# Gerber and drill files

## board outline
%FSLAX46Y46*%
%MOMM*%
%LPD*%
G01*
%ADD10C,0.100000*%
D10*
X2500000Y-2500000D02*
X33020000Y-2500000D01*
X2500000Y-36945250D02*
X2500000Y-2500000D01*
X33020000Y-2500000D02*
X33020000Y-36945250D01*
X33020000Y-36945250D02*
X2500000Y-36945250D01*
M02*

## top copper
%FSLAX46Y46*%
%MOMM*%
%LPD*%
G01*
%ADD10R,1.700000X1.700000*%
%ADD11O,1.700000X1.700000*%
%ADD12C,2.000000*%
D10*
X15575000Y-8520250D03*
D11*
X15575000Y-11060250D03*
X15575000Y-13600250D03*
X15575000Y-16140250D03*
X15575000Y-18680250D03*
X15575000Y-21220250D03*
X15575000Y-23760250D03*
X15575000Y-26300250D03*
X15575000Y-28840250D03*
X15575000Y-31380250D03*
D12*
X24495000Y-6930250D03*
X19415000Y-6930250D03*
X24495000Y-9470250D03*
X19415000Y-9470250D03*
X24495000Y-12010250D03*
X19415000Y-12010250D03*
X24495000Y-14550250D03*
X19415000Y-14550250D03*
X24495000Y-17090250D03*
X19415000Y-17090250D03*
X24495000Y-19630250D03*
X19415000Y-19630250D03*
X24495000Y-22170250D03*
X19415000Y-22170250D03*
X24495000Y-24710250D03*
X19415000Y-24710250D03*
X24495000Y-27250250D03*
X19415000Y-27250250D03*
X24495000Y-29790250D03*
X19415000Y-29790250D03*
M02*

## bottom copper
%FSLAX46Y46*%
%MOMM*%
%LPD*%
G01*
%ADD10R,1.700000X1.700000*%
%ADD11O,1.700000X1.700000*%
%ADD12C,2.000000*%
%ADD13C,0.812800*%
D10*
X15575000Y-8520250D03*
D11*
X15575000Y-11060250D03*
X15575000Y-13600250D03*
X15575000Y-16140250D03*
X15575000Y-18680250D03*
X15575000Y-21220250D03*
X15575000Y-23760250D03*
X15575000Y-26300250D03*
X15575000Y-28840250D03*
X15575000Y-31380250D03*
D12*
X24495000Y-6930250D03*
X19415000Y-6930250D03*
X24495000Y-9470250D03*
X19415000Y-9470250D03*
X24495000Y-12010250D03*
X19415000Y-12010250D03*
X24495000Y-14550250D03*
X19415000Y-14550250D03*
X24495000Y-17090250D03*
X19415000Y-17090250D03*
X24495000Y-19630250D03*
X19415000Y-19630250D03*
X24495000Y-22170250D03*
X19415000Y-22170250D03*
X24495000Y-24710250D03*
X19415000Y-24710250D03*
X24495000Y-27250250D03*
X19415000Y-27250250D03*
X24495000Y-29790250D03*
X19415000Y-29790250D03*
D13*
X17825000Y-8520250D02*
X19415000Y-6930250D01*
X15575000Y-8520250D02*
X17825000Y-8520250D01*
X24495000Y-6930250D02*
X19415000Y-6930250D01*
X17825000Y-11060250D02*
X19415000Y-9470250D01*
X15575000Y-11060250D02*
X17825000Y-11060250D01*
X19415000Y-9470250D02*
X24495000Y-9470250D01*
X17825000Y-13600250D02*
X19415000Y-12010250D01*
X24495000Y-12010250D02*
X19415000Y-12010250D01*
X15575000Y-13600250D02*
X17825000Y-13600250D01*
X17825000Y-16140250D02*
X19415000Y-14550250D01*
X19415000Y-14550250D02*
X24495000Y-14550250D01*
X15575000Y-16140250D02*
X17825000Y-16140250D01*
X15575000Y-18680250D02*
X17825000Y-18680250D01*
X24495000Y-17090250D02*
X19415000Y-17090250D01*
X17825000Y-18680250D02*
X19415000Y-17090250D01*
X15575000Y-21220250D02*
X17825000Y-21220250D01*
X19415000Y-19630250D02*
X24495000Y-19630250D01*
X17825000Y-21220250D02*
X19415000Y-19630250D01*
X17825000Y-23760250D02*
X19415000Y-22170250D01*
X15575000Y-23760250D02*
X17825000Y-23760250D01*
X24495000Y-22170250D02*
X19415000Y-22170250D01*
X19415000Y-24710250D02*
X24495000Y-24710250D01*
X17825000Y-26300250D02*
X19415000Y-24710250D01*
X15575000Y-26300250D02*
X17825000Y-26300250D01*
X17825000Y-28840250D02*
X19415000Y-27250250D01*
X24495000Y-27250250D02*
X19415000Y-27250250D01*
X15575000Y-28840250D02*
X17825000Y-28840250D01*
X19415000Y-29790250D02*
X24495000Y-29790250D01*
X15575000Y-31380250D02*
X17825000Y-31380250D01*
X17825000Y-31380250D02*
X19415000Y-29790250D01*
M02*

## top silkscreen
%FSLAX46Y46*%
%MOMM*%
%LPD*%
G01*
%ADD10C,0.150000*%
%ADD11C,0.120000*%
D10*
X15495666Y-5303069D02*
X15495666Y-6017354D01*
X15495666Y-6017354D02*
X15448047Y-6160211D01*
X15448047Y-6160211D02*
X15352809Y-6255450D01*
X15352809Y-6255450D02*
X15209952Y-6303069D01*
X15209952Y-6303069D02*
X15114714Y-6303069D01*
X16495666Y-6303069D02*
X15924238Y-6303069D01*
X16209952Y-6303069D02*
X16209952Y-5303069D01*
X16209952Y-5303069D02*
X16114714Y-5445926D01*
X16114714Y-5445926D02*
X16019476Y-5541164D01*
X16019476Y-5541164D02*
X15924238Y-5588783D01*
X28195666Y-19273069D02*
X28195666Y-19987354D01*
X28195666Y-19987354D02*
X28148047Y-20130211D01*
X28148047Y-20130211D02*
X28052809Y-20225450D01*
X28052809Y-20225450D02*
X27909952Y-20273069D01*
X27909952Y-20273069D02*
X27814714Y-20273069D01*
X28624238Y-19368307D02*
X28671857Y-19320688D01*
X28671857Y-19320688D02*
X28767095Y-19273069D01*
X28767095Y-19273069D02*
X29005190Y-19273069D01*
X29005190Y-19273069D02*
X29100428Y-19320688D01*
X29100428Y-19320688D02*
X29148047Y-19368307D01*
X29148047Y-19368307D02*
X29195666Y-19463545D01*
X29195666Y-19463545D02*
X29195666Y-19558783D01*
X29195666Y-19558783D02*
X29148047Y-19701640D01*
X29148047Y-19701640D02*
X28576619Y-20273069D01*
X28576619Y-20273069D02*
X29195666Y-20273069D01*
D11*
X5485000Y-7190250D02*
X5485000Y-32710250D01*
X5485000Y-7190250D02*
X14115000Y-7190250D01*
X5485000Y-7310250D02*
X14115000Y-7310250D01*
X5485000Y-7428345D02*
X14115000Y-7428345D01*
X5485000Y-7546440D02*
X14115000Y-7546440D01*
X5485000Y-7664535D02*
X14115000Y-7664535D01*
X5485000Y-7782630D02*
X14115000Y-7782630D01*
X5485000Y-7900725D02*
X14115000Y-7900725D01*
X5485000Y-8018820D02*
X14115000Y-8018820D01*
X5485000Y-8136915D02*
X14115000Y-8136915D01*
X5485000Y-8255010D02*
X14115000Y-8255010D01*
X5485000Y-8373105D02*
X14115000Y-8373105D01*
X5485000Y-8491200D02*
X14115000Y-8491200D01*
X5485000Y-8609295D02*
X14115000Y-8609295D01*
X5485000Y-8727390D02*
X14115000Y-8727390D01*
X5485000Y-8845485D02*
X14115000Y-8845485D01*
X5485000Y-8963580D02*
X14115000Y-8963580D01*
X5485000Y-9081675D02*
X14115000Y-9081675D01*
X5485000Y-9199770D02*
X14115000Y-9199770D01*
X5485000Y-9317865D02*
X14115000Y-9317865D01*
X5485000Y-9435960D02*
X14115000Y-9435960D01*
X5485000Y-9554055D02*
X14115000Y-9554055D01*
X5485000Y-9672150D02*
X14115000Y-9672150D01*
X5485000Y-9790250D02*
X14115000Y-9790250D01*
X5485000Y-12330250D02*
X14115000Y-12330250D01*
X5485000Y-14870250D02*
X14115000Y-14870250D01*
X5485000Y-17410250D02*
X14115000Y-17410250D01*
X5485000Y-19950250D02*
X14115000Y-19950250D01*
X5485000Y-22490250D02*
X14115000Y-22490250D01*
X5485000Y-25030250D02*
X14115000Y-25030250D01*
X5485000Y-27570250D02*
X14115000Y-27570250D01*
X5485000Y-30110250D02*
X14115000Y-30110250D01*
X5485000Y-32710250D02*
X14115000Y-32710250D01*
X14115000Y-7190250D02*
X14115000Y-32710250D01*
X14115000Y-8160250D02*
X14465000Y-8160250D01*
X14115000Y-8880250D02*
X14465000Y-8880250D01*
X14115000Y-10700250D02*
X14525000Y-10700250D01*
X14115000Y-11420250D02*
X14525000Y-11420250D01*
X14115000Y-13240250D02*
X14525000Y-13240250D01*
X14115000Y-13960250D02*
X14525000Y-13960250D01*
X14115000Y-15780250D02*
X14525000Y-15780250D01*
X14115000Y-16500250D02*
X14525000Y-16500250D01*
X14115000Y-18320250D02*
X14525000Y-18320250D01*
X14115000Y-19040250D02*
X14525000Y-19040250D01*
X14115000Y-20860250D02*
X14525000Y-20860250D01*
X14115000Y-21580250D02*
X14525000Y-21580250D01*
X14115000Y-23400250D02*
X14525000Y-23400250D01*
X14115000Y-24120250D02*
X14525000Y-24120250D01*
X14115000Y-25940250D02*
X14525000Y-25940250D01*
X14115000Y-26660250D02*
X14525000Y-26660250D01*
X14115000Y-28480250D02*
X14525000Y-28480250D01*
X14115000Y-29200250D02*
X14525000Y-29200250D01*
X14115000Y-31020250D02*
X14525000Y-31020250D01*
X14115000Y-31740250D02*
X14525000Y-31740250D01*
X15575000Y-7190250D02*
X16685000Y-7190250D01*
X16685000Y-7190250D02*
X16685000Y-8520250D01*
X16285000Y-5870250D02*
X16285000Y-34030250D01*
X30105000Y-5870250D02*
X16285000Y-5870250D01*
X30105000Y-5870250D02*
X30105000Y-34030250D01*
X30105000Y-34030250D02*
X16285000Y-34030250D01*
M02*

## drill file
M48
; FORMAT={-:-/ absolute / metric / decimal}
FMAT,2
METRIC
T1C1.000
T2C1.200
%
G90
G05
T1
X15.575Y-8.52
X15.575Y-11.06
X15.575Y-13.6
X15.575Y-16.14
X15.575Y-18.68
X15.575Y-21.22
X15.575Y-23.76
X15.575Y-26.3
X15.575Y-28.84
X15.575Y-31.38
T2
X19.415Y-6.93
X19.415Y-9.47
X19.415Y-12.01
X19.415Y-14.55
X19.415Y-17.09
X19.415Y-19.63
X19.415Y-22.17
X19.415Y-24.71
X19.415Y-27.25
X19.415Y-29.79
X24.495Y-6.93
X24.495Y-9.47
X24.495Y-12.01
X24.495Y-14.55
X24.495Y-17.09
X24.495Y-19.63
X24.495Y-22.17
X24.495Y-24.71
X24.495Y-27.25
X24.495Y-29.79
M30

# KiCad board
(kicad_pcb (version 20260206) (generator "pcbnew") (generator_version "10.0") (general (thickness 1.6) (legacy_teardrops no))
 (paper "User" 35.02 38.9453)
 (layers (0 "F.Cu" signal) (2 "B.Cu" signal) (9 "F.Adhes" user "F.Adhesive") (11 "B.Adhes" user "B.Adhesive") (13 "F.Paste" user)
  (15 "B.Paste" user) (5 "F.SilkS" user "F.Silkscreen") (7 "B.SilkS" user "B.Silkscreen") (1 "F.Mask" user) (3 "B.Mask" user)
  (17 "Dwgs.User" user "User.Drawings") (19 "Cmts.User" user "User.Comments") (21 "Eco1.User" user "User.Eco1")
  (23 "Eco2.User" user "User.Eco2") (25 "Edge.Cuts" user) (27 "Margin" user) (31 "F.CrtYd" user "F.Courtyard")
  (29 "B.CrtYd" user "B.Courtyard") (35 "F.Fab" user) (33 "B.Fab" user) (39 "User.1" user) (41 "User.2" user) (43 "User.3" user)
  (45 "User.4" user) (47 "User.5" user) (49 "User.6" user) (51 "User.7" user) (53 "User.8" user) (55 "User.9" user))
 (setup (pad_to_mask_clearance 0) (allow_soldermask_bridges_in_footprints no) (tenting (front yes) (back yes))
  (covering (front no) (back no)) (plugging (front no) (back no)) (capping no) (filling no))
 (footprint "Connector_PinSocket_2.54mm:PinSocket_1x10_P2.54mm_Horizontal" (layer "F.Cu") (at 15.575 8.52025)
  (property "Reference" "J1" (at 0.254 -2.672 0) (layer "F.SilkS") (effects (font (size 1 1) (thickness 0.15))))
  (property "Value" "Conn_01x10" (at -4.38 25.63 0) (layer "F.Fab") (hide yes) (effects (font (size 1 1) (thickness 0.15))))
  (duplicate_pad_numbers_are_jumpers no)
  (fp_line (start -10.09 -1.33) (end -10.09 24.19) (stroke (width 0.12) (type solid)) (layer "F.SilkS"))
  (fp_line (start -10.09 -1.33) (end -1.46 -1.33) (stroke (width 0.12) (type solid)) (layer "F.SilkS"))
  (fp_line (start -10.09 -1.21) (end -1.46 -1.21) (stroke (width 0.12) (type solid)) (layer "F.SilkS"))
  (fp_line (start -10.09 -1.091905) (end -1.46 -1.091905) (stroke (width 0.12) (type solid)) (layer "F.SilkS"))
  (fp_line (start -10.09 -0.97381) (end -1.46 -0.97381) (stroke (width 0.12) (type solid)) (layer "F.SilkS"))
  (fp_line (start -10.09 -0.855715) (end -1.46 -0.855715) (stroke (width 0.12) (type solid)) (layer "F.SilkS"))
  (fp_line (start -10.09 -0.73762) (end -1.46 -0.73762) (stroke (width 0.12) (type solid)) (layer "F.SilkS"))
  (fp_line (start -10.09 -0.619525) (end -1.46 -0.619525) (stroke (width 0.12) (type solid)) (layer "F.SilkS"))
  (fp_line (start -10.09 -0.50143) (end -1.46 -0.50143) (stroke (width 0.12) (type solid)) (layer "F.SilkS"))
  (fp_line (start -10.09 -0.383335) (end -1.46 -0.383335) (stroke (width 0.12) (type solid)) (layer "F.SilkS"))
  (fp_line (start -10.09 -0.26524) (end -1.46 -0.26524) (stroke (width 0.12) (type solid)) (layer "F.SilkS"))
  (fp_line (start -10.09 -0.147145) (end -1.46 -0.147145) (stroke (width 0.12) (type solid)) (layer "F.SilkS"))
  (fp_line (start -10.09 -0.02905) (end -1.46 -0.02905) (stroke (width 0.12) (type solid)) (layer "F.SilkS"))
  (fp_line (start -10.09 0.089045) (end -1.46 0.089045) (stroke (width 0.12) (type solid)) (layer "F.SilkS"))
  (fp_line (start -10.09 0.20714) (end -1.46 0.20714) (stroke (width 0.12) (type solid)) (layer "F.SilkS"))
  (fp_line (start -10.09 0.325235) (end -1.46 0.325235) (stroke (width 0.12) (type solid)) (layer "F.SilkS"))
  (fp_line (start -10.09 0.44333) (end -1.46 0.44333) (stroke (width 0.12) (type solid)) (layer "F.SilkS"))
  (fp_line (start -10.09 0.561425) (end -1.46 0.561425) (stroke (width 0.12) (type solid)) (layer "F.SilkS"))
  (fp_line (start -10.09 0.67952) (end -1.46 0.67952) (stroke (width 0.12) (type solid)) (layer "F.SilkS"))
  (fp_line (start -10.09 0.797615) (end -1.46 0.797615) (stroke (width 0.12) (type solid)) (layer "F.SilkS"))
  (fp_line (start -10.09 0.91571) (end -1.46 0.91571) (stroke (width 0.12) (type solid)) (layer "F.SilkS"))
  (fp_line (start -10.09 1.033805) (end -1.46 1.033805) (stroke (width 0.12) (type solid)) (layer "F.SilkS"))
  (fp_line (start -10.09 1.1519) (end -1.46 1.1519) (stroke (width 0.12) (type solid)) (layer "F.SilkS"))
  (fp_line (start -10.09 1.27) (end -1.46 1.27) (stroke (width 0.12) (type solid)) (layer "F.SilkS"))
  (fp_line (start -10.09 3.81) (end -1.46 3.81) (stroke (width 0.12) (type solid)) (layer "F.SilkS"))
  (fp_line (start -10.09 6.35) (end -1.46 6.35) (stroke (width 0.12) (type solid)) (layer "F.SilkS"))
  (fp_line (start -10.09 8.89) (end -1.46 8.89) (stroke (width 0.12) (type solid)) (layer "F.SilkS"))
  (fp_line (start -10.09 11.43) (end -1.46 11.43) (stroke (width 0.12) (type solid)) (layer "F.SilkS"))
  (fp_line (start -10.09 13.97) (end -1.46 13.97) (stroke (width 0.12) (type solid)) (layer "F.SilkS"))
  (fp_line (start -10.09 16.51) (end -1.46 16.51) (stroke (width 0.12) (type solid)) (layer "F.SilkS"))
  (fp_line (start -10.09 19.05) (end -1.46 19.05) (stroke (width 0.12) (type solid)) (layer "F.SilkS"))
  (fp_line (start -10.09 21.59) (end -1.46 21.59) (stroke (width 0.12) (type solid)) (layer "F.SilkS"))
  (fp_line (start -10.09 24.19) (end -1.46 24.19) (stroke (width 0.12) (type solid)) (layer "F.SilkS"))
  (fp_line (start -1.46 -1.33) (end -1.46 24.19) (stroke (width 0.12) (type solid)) (layer "F.SilkS"))
  (fp_line (start -1.46 -0.36) (end -1.11 -0.36) (stroke (width 0.12) (type solid)) (layer "F.SilkS"))
  (fp_line (start -1.46 0.36) (end -1.11 0.36) (stroke (width 0.12) (type solid)) (layer "F.SilkS"))
  (fp_line (start -1.46 2.18) (end -1.05 2.18) (stroke (width 0.12) (type solid)) (layer "F.SilkS"))
  (fp_line (start -1.46 2.9) (end -1.05 2.9) (stroke (width 0.12) (type solid)) (layer "F.SilkS"))
  (fp_line (start -1.46 4.72) (end -1.05 4.72) (stroke (width 0.12) (type solid)) (layer "F.SilkS"))
  (fp_line (start -1.46 5.44) (end -1.05 5.44) (stroke (width 0.12) (type solid)) (layer "F.SilkS"))
  (fp_line (start -1.46 7.26) (end -1.05 7.26) (stroke (width 0.12) (type solid)) (layer "F.SilkS"))
  (fp_line (start -1.46 7.98) (end -1.05 7.98) (stroke (width 0.12) (type solid)) (layer "F.SilkS"))
  (fp_line (start -1.46 9.8) (end -1.05 9.8) (stroke (width 0.12) (type solid)) (layer "F.SilkS"))
  (fp_line (start -1.46 10.52) (end -1.05 10.52) (stroke (width 0.12) (type solid)) (layer "F.SilkS"))
  (fp_line (start -1.46 12.34) (end -1.05 12.34) (stroke (width 0.12) (type solid)) (layer "F.SilkS"))
  (fp_line (start -1.46 13.06) (end -1.05 13.06) (stroke (width 0.12) (type solid)) (layer "F.SilkS"))
  (fp_line (start -1.46 14.88) (end -1.05 14.88) (stroke (width 0.12) (type solid)) (layer "F.SilkS"))
  (fp_line (start -1.46 15.6) (end -1.05 15.6) (stroke (width 0.12) (type solid)) (layer "F.SilkS"))
  (fp_line (start -1.46 17.42) (end -1.05 17.42) (stroke (width 0.12) (type solid)) (layer "F.SilkS"))
  (fp_line (start -1.46 18.14) (end -1.05 18.14) (stroke (width 0.12) (type solid)) (layer "F.SilkS"))
  (fp_line (start -1.46 19.96) (end -1.05 19.96) (stroke (width 0.12) (type solid)) (layer "F.SilkS"))
  (fp_line (start -1.46 20.68) (end -1.05 20.68) (stroke (width 0.12) (type solid)) (layer "F.SilkS"))
  (fp_line (start -1.46 22.5) (end -1.05 22.5) (stroke (width 0.12) (type solid)) (layer "F.SilkS"))
  (fp_line (start -1.46 23.22) (end -1.05 23.22) (stroke (width 0.12) (type solid)) (layer "F.SilkS"))
  (fp_line (start 0 -1.33) (end 1.11 -1.33) (stroke (width 0.12) (type solid)) (layer "F.SilkS"))
  (fp_line (start 1.11 -1.33) (end 1.11 0) (stroke (width 0.12) (type solid)) (layer "F.SilkS"))
  (pad "1" thru_hole rect (at 0 0) (size 1.7 1.7) (drill 1) (layers "*.Cu" "*.Mask") (remove_unused_layers no) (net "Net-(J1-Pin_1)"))
  (pad "2" thru_hole oval (at 0 2.54) (size 1.7 1.7) (drill 1) (layers "*.Cu" "*.Mask") (remove_unused_layers no) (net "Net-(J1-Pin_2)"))
  (pad "3" thru_hole oval (at 0 5.08) (size 1.7 1.7) (drill 1) (layers "*.Cu" "*.Mask") (remove_unused_layers no) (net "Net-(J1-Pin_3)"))
  (pad "4" thru_hole oval (at 0 7.62) (size 1.7 1.7) (drill 1) (layers "*.Cu" "*.Mask") (remove_unused_layers no) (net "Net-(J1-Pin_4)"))
  (pad "5" thru_hole oval (at 0 10.16) (size 1.7 1.7) (drill 1) (layers "*.Cu" "*.Mask") (remove_unused_layers no) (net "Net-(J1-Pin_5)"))
  (pad "6" thru_hole oval (at 0 12.7) (size 1.7 1.7) (drill 1) (layers "*.Cu" "*.Mask") (remove_unused_layers no) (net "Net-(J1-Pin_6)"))
  (pad "7" thru_hole oval (at 0 15.24) (size 1.7 1.7) (drill 1) (layers "*.Cu" "*.Mask") (remove_unused_layers no) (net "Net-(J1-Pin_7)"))
  (pad "8" thru_hole oval (at 0 17.78) (size 1.7 1.7) (drill 1) (layers "*.Cu" "*.Mask") (remove_unused_layers no) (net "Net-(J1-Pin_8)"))
  (pad "9" thru_hole oval (at 0 20.32) (size 1.7 1.7) (drill 1) (layers "*.Cu" "*.Mask") (remove_unused_layers no) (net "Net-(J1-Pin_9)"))
  (pad "10" thru_hole oval (at 0 22.86) (size 1.7 1.7) (drill 1) (layers "*.Cu" "*.Mask") (remove_unused_layers no) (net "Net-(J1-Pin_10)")))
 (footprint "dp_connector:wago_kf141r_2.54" (layer "F.Cu") (at 23.195 19.95025 -90)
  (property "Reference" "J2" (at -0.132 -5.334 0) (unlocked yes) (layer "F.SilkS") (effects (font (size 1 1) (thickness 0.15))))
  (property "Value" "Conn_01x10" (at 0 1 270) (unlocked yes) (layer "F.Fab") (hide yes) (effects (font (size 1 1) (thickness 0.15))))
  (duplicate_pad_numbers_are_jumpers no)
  (fp_line (start -14.08 6.91) (end 14.08 6.91) (stroke (width 0.12) (type default)) (layer "F.SilkS"))
  (fp_line (start -14.08 -6.91) (end -14.08 6.91) (stroke (width 0.12) (type default)) (layer "F.SilkS"))
  (fp_line (start -14.08 -6.91) (end 14.08 -6.91) (stroke (width 0.12) (type default)) (layer "F.SilkS"))
  (fp_line (start 14.08 -6.91) (end 14.08 6.91) (stroke (width 0.12) (type default)) (layer "F.SilkS"))
  (pad "1" thru_hole circle (at -13.02 -1.3 270) (size 2 2) (drill 1.2) (layers "*.Cu" "*.Mask") (remove_unused_layers no)
   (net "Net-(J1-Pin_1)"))
  (pad "1" thru_hole circle (at -13.02 3.78 270) (size 2 2) (drill 1.2) (layers "*.Cu" "*.Mask") (remove_unused_layers no)
   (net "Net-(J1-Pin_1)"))
  (pad "2" thru_hole circle (at -10.48 -1.3 270) (size 2 2) (drill 1.2) (layers "*.Cu" "*.Mask") (remove_unused_layers no)
   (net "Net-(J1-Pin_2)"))
  (pad "2" thru_hole circle (at -10.48 3.78 270) (size 2 2) (drill 1.2) (layers "*.Cu" "*.Mask") (remove_unused_layers no)
   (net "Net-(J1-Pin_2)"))
  (pad "3" thru_hole circle (at -7.94 -1.3 270) (size 2 2) (drill 1.2) (layers "*.Cu" "*.Mask") (remove_unused_layers no)
   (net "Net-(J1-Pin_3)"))
  (pad "3" thru_hole circle (at -7.94 3.78 270) (size 2 2) (drill 1.2) (layers "*.Cu" "*.Mask") (remove_unused_layers no)
   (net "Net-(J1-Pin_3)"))
  (pad "4" thru_hole circle (at -5.4 -1.3 270) (size 2 2) (drill 1.2) (layers "*.Cu" "*.Mask") (remove_unused_layers no)
   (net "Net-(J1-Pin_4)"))
  (pad "4" thru_hole circle (at -5.4 3.78 270) (size 2 2) (drill 1.2) (layers "*.Cu" "*.Mask") (remove_unused_layers no)
   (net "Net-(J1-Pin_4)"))
  (pad "5" thru_hole circle (at -2.86 -1.3 270) (size 2 2) (drill 1.2) (layers "*.Cu" "*.Mask") (remove_unused_layers no)
   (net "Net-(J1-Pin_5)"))
  (pad "5" thru_hole circle (at -2.86 3.78 270) (size 2 2) (drill 1.2) (layers "*.Cu" "*.Mask") (remove_unused_layers no)
   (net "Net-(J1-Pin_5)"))
  (pad "6" thru_hole circle (at -0.32 -1.3 270) (size 2 2) (drill 1.2) (layers "*.Cu" "*.Mask") (remove_unused_layers no)
   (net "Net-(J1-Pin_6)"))
  (pad "6" thru_hole circle (at -0.32 3.78 270) (size 2 2) (drill 1.2) (layers "*.Cu" "*.Mask") (remove_unused_layers no)
   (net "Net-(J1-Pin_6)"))
  (pad "7" thru_hole circle (at 2.22 -1.3 270) (size 2 2) (drill 1.2) (layers "*.Cu" "*.Mask") (remove_unused_layers no)
   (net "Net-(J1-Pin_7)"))
  (pad "7" thru_hole circle (at 2.22 3.78 270) (size 2 2) (drill 1.2) (layers "*.Cu" "*.Mask") (remove_unused_layers no)
   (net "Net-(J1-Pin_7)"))
  (pad "8" thru_hole circle (at 4.76 -1.3 270) (size 2 2) (drill 1.2) (layers "*.Cu" "*.Mask") (remove_unused_layers no)
   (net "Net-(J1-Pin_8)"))
  (pad "8" thru_hole circle (at 4.76 3.78 270) (size 2 2) (drill 1.2) (layers "*.Cu" "*.Mask") (remove_unused_layers no)
   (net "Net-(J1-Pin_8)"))
  (pad "9" thru_hole circle (at 7.3 -1.3 270) (size 2 2) (drill 1.2) (layers "*.Cu" "*.Mask") (remove_unused_layers no)
   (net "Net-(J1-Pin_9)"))
  (pad "9" thru_hole circle (at 7.3 3.78 270) (size 2 2) (drill 1.2) (layers "*.Cu" "*.Mask") (remove_unused_layers no)
   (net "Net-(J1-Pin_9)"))
  (pad "10" thru_hole circle (at 9.84 -1.3 270) (size 2 2) (drill 1.2) (layers "*.Cu" "*.Mask") (remove_unused_layers no)
   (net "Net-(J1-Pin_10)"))
  (pad "10" thru_hole circle (at 9.84 3.78 270) (size 2 2) (drill 1.2) (layers "*.Cu" "*.Mask") (remove_unused_layers no)
   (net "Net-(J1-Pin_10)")))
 (gr_line (start 2.5 2.5) (end 33.02 2.5) (stroke (width 0.1) (type default)) (layer "Edge.Cuts"))
 (gr_line (start 2.5 36.94525) (end 2.5 2.5) (stroke (width 0.1) (type default)) (layer "Edge.Cuts"))
 (gr_line (start 33.02 2.5) (end 33.02 36.94525) (stroke (width 0.1) (type default)) (layer "Edge.Cuts"))
 (gr_line (start 33.02 36.94525) (end 2.5 36.94525) (stroke (width 0.1) (type default)) (layer "Edge.Cuts"))
 (segment (start 17.825 8.52025) (end 19.415 6.93025) (width 0.8128) (layer "B.Cu") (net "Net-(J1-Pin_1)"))
 (segment (start 15.575 8.52025) (end 17.825 8.52025) (width 0.8128) (layer "B.Cu") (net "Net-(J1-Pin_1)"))
 (segment (start 24.495 6.93025) (end 19.415 6.93025) (width 0.8128) (layer "B.Cu") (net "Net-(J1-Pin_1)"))
 (segment (start 17.825 11.06025) (end 19.415 9.47025) (width 0.8128) (layer "B.Cu") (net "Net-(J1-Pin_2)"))
 (segment (start 15.575 11.06025) (end 17.825 11.06025) (width 0.8128) (layer "B.Cu") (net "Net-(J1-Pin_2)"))
 (segment (start 19.415 9.47025) (end 24.495 9.47025) (width 0.8128) (layer "B.Cu") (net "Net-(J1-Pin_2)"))
 (segment (start 17.825 13.60025) (end 19.415 12.01025) (width 0.8128) (layer "B.Cu") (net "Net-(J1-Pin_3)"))
 (segment (start 24.495 12.01025) (end 19.415 12.01025) (width 0.8128) (layer "B.Cu") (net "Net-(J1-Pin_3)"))
 (segment (start 15.575 13.60025) (end 17.825 13.60025) (width 0.8128) (layer "B.Cu") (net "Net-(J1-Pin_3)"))
 (segment (start 17.825 16.14025) (end 19.415 14.55025) (width 0.8128) (layer "B.Cu") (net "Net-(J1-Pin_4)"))
 (segment (start 19.415 14.55025) (end 24.495 14.55025) (width 0.8128) (layer "B.Cu") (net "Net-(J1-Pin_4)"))
 (segment (start 15.575 16.14025) (end 17.825 16.14025) (width 0.8128) (layer "B.Cu") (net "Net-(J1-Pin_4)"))
 (segment (start 15.575 18.68025) (end 17.825 18.68025) (width 0.8128) (layer "B.Cu") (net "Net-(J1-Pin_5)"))
 (segment (start 24.495 17.09025) (end 19.415 17.09025) (width 0.8128) (layer "B.Cu") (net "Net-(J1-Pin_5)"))
 (segment (start 17.825 18.68025) (end 19.415 17.09025) (width 0.8128) (layer "B.Cu") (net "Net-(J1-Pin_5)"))
 (segment (start 15.575 21.22025) (end 17.825 21.22025) (width 0.8128) (layer "B.Cu") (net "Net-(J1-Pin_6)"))
 (segment (start 19.415 19.63025) (end 24.495 19.63025) (width 0.8128) (layer "B.Cu") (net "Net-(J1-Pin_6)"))
 (segment (start 17.825 21.22025) (end 19.415 19.63025) (width 0.8128) (layer "B.Cu") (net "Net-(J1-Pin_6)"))
 (segment (start 17.825 23.76025) (end 19.415 22.17025) (width 0.8128) (layer "B.Cu") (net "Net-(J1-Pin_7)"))
 (segment (start 15.575 23.76025) (end 17.825 23.76025) (width 0.8128) (layer "B.Cu") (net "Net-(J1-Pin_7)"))
 (segment (start 24.495 22.17025) (end 19.415 22.17025) (width 0.8128) (layer "B.Cu") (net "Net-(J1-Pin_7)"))
 (segment (start 19.415 24.71025) (end 24.495 24.71025) (width 0.8128) (layer "B.Cu") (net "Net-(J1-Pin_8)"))
 (segment (start 17.825 26.30025) (end 19.415 24.71025) (width 0.8128) (layer "B.Cu") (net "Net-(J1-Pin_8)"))
 (segment (start 15.575 26.30025) (end 17.825 26.30025) (width 0.8128) (layer "B.Cu") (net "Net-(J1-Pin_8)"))
 (segment (start 17.825 28.84025) (end 19.415 27.25025) (width 0.8128) (layer "B.Cu") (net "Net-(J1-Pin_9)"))
 (segment (start 24.495 27.25025) (end 19.415 27.25025) (width 0.8128) (layer "B.Cu") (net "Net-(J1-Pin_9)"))
 (segment (start 15.575 28.84025) (end 17.825 28.84025) (width 0.8128) (layer "B.Cu") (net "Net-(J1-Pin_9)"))
 (segment (start 19.415 29.79025) (end 24.495 29.79025) (width 0.8128) (layer "B.Cu") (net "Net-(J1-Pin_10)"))
 (segment (start 15.575 31.38025) (end 17.825 31.38025) (width 0.8128) (layer "B.Cu") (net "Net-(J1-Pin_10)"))
 (segment (start 17.825 31.38025) (end 19.415 29.79025) (width 0.8128) (layer "B.Cu") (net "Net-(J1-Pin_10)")))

